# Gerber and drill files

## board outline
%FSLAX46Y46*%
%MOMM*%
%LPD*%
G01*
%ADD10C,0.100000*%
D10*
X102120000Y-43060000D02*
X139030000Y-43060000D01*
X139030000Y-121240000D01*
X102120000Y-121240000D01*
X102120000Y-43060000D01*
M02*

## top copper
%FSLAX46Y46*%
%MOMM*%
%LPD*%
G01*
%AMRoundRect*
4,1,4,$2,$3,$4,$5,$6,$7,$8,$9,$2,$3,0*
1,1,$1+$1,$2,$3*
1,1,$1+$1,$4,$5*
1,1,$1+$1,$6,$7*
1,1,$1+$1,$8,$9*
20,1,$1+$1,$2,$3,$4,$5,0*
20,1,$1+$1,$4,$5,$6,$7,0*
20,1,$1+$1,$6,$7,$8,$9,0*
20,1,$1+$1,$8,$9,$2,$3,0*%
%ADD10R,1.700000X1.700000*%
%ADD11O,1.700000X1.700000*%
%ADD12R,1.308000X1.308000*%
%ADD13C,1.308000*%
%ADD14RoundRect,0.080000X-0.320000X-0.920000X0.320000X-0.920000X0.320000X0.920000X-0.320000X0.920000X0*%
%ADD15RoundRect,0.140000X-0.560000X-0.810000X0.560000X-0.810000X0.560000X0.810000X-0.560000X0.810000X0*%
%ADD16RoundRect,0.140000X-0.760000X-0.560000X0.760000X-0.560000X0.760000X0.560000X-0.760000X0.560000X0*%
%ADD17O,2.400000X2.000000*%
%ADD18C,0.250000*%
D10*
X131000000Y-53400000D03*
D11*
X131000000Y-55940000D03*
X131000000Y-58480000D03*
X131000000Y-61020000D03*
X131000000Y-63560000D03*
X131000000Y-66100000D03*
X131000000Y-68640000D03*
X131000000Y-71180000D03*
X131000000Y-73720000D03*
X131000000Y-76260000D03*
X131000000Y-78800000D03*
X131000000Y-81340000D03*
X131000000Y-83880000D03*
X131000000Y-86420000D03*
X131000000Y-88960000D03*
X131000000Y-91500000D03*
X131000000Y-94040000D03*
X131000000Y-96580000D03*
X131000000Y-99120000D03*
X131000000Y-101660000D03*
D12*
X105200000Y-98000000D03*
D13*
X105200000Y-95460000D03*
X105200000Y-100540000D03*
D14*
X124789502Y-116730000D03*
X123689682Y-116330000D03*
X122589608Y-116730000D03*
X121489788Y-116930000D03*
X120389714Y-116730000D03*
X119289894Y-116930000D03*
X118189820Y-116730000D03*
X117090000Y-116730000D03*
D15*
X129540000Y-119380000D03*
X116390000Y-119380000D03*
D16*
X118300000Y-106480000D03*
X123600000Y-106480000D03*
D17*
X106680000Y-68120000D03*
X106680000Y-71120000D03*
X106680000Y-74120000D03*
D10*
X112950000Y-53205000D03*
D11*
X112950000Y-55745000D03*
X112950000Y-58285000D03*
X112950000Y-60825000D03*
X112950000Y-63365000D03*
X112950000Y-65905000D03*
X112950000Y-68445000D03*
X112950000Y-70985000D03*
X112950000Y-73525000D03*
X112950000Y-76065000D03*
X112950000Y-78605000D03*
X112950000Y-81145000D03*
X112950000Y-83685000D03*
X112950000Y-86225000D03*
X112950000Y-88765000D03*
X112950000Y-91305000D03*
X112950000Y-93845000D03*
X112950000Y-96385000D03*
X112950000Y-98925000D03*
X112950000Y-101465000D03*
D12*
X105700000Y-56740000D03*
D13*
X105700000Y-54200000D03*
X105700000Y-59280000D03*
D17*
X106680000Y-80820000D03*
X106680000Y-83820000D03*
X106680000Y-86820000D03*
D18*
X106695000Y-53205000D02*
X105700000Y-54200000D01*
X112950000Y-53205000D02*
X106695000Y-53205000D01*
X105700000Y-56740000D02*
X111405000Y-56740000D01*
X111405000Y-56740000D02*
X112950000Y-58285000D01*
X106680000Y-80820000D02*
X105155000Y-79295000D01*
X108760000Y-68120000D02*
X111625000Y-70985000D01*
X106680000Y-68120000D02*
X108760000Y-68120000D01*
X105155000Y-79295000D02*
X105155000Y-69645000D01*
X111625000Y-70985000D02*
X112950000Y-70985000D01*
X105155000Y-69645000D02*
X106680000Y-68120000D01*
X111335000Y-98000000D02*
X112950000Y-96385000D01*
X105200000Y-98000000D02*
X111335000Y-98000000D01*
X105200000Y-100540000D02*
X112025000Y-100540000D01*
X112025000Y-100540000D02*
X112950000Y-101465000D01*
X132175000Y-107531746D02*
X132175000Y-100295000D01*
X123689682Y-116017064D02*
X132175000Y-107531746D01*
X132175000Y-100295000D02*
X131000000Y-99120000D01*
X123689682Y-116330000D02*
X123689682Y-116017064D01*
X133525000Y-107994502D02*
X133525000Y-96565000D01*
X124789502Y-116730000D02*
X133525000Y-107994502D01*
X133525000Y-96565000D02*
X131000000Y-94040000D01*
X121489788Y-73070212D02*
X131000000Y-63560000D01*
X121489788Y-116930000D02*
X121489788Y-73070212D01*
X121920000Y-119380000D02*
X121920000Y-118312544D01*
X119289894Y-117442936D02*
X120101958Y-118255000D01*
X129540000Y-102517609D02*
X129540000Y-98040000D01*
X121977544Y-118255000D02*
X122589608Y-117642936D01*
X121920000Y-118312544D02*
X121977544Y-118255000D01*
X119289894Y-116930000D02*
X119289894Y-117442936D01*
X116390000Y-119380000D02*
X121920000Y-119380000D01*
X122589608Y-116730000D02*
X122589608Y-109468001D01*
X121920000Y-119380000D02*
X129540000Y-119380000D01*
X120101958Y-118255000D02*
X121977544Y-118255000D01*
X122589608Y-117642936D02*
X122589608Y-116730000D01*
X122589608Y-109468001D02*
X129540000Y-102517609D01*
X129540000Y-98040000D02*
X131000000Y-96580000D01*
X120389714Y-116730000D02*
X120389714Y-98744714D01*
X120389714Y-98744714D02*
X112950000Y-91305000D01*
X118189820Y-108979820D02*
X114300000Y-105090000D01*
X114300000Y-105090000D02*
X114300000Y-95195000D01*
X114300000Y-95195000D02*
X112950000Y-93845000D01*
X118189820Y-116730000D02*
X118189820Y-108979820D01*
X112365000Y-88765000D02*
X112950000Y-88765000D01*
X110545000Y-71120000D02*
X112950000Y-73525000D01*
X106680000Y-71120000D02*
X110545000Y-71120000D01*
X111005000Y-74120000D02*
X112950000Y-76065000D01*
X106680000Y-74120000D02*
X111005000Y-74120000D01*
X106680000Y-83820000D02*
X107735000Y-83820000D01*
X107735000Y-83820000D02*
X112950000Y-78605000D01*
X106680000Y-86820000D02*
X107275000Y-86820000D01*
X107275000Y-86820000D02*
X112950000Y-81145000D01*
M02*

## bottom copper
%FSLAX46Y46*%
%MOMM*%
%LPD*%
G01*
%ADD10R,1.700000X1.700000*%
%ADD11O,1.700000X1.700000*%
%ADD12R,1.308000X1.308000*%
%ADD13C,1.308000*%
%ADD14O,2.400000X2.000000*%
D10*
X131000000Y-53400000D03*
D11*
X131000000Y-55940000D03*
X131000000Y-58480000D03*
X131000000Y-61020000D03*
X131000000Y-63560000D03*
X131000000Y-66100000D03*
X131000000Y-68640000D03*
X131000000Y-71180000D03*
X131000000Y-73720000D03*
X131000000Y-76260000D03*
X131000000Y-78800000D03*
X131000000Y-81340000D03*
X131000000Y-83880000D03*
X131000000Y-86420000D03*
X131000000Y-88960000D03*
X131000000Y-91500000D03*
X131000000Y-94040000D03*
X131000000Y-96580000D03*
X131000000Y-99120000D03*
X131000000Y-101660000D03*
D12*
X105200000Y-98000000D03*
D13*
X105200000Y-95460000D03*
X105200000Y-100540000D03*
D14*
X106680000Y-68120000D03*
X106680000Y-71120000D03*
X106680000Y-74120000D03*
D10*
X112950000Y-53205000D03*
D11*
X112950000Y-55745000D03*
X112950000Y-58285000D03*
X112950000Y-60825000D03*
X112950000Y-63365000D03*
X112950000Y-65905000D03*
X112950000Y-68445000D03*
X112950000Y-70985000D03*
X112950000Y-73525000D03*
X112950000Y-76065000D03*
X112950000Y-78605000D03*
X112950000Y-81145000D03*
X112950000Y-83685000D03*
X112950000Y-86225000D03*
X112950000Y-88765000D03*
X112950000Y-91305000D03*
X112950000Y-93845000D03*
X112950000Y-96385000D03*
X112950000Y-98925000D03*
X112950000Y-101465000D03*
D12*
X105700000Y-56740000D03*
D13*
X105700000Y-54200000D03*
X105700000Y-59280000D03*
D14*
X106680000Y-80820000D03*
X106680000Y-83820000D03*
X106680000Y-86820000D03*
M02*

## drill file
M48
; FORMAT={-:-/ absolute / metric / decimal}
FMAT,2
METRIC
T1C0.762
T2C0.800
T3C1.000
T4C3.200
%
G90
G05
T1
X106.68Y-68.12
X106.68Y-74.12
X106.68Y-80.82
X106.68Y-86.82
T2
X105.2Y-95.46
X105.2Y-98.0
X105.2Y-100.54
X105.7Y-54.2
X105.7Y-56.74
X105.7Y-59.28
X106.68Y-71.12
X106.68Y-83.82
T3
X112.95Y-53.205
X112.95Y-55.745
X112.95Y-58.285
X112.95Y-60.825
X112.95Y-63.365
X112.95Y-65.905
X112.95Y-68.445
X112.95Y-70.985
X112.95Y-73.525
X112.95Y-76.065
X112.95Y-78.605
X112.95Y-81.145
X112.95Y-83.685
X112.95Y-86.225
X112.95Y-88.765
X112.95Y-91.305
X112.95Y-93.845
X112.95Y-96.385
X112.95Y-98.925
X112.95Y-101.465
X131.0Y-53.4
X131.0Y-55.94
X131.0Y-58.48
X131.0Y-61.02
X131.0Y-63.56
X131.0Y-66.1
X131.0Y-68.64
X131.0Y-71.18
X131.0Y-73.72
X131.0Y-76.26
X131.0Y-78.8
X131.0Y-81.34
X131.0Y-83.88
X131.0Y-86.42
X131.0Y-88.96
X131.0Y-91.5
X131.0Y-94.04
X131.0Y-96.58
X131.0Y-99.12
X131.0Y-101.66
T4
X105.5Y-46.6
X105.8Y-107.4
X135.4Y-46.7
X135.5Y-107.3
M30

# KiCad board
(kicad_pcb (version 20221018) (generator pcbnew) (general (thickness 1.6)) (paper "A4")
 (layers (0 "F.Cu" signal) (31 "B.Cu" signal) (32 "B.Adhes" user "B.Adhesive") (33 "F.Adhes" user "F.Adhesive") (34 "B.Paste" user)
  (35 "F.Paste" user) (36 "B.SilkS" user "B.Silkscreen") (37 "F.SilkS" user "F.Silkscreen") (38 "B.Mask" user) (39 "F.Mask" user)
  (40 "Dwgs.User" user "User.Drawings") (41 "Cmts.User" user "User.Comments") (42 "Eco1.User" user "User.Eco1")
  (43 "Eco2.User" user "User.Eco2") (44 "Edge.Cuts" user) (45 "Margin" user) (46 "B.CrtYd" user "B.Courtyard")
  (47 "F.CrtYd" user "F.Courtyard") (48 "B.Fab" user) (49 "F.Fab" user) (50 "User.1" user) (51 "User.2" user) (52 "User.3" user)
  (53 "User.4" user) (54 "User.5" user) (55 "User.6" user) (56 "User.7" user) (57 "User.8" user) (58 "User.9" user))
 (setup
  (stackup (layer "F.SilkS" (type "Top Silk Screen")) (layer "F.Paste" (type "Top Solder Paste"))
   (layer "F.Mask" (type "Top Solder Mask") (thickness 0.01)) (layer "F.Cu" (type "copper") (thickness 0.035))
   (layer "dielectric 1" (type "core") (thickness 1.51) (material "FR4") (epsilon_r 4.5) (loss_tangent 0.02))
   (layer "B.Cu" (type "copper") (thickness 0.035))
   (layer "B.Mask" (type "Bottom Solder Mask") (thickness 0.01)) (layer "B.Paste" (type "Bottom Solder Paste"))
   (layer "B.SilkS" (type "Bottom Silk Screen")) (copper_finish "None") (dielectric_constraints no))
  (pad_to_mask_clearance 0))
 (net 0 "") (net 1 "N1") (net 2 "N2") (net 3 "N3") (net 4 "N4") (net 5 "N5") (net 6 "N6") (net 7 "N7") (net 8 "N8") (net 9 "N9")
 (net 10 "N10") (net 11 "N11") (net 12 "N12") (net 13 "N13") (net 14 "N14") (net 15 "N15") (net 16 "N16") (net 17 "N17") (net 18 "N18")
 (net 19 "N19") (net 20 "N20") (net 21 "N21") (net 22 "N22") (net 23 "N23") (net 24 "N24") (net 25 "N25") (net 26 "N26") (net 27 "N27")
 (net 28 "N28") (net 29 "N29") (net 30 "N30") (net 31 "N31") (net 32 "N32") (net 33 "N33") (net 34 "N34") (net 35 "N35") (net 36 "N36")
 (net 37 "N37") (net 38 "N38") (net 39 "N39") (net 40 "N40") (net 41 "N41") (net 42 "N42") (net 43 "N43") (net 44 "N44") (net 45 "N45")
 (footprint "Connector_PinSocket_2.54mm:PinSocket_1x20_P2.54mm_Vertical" (layer "F.Cu") (at 131 53.4)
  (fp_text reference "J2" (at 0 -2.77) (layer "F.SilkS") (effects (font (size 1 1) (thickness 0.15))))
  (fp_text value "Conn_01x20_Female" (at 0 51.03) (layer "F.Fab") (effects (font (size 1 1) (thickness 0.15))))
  (pad "1" thru_hole rect (at 0 0) (size 1.7 1.7) (drill 1) (layers "*.Cu" "*.Mask") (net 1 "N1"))
  (pad "2" thru_hole oval (at 0 2.54) (size 1.7 1.7) (drill 1) (layers "*.Cu" "*.Mask") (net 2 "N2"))
  (pad "3" thru_hole oval (at 0 5.08) (size 1.7 1.7) (drill 1) (layers "*.Cu" "*.Mask") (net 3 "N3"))
  (pad "4" thru_hole oval (at 0 7.62) (size 1.7 1.7) (drill 1) (layers "*.Cu" "*.Mask") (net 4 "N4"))
  (pad "5" thru_hole oval (at 0 10.16) (size 1.7 1.7) (drill 1) (layers "*.Cu" "*.Mask") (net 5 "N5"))
  (pad "6" thru_hole oval (at 0 12.7) (size 1.7 1.7) (drill 1) (layers "*.Cu" "*.Mask") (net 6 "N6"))
  (pad "7" thru_hole oval (at 0 15.24) (size 1.7 1.7) (drill 1) (layers "*.Cu" "*.Mask") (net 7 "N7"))
  (pad "8" thru_hole oval (at 0 17.78) (size 1.7 1.7) (drill 1) (layers "*.Cu" "*.Mask") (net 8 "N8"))
  (pad "9" thru_hole oval (at 0 20.32) (size 1.7 1.7) (drill 1) (layers "*.Cu" "*.Mask") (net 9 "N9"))
  (pad "10" thru_hole oval (at 0 22.86) (size 1.7 1.7) (drill 1) (layers "*.Cu" "*.Mask") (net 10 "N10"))
  (pad "11" thru_hole oval (at 0 25.4) (size 1.7 1.7) (drill 1) (layers "*.Cu" "*.Mask") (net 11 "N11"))
  (pad "12" thru_hole oval (at 0 27.94) (size 1.7 1.7) (drill 1) (layers "*.Cu" "*.Mask") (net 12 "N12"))
  (pad "13" thru_hole oval (at 0 30.48) (size 1.7 1.7) (drill 1) (layers "*.Cu" "*.Mask") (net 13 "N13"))
  (pad "14" thru_hole oval (at 0 33.02) (size 1.7 1.7) (drill 1) (layers "*.Cu" "*.Mask") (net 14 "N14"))
  (pad "15" thru_hole oval (at 0 35.56) (size 1.7 1.7) (drill 1) (layers "*.Cu" "*.Mask") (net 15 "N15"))
  (pad "16" thru_hole oval (at 0 38.1) (size 1.7 1.7) (drill 1) (layers "*.Cu" "*.Mask") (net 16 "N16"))
  (pad "17" thru_hole oval (at 0 40.64) (size 1.7 1.7) (drill 1) (layers "*.Cu" "*.Mask") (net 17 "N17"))
  (pad "18" thru_hole oval (at 0 43.18) (size 1.7 1.7) (drill 1) (layers "*.Cu" "*.Mask") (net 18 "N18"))
  (pad "19" thru_hole oval (at 0 45.72) (size 1.7 1.7) (drill 1) (layers "*.Cu" "*.Mask") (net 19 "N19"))
  (pad "20" thru_hole oval (at 0 48.26) (size 1.7 1.7) (drill 1) (layers "*.Cu" "*.Mask") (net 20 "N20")))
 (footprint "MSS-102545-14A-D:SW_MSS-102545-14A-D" (layer "F.Cu") (at 105.2 98 -90)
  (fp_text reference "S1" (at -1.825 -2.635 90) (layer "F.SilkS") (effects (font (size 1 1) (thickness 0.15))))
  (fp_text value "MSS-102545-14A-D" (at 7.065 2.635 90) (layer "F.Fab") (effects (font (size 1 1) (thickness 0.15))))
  (pad "1" thru_hole rect (at 0 0 270) (size 1.308 1.308) (drill 0.8) (layers "*.Cu" "*.Mask") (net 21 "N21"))
  (pad "2" thru_hole circle (at -2.54 0 270) (size 1.308 1.308) (drill 0.8) (layers "*.Cu" "*.Mask") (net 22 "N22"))
  (pad "3" thru_hole circle (at 2.54 0 270) (size 1.308 1.308) (drill 0.8) (layers "*.Cu" "*.Mask") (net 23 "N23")))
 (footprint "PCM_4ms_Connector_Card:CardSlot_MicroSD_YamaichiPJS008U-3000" (layer "F.Cu") (at 121.92 117.83008)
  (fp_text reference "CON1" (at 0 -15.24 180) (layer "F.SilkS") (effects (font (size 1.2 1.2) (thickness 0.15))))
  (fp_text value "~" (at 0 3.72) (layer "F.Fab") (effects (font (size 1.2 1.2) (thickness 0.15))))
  (pad "1" smd roundrect (at 2.869502 -1.10008) (size 0.8 2) (layers "F.Cu" "F.Paste" "F.Mask") (roundrect_rratio 0.1) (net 17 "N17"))
  (pad "2" smd roundrect (at 1.769682 -1.50008) (size 0.8 2) (layers "F.Cu" "F.Paste" "F.Mask") (roundrect_rratio 0.1) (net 19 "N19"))
  (pad "3" smd roundrect (at 0.669608 -1.10008) (size 0.8 2) (layers "F.Cu" "F.Paste" "F.Mask") (roundrect_rratio 0.1) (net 18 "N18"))
  (pad "4" smd roundrect (at -0.430212 -0.90008) (size 0.8 2) (layers "F.Cu" "F.Paste" "F.Mask") (roundrect_rratio 0.1) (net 5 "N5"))
  (pad "5" smd roundrect (at -1.530286 -1.10008) (size 0.8 2) (layers "F.Cu" "F.Paste" "F.Mask") (roundrect_rratio 0.1) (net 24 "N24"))
  (pad "6" smd roundrect (at -2.630106 -0.90008) (size 0.8 2) (layers "F.Cu" "F.Paste" "F.Mask") (roundrect_rratio 0.1) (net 18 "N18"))
  (pad "7" smd roundrect (at -3.73018 -1.10008) (size 0.8 2) (layers "F.Cu" "F.Paste" "F.Mask") (roundrect_rratio 0.1) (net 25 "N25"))
  (pad "8" smd roundrect (at -4.83 -1.10008) (size 0.8 2) (layers "F.Cu" "F.Paste" "F.Mask") (roundrect_rratio 0.1) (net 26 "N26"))
  (pad "9" smd roundrect (at 7.62 1.54992) (size 1.4 1.9) (layers "F.Cu" "F.Paste" "F.Mask") (roundrect_rratio 0.1) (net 18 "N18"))
  (pad "10" smd roundrect (at -5.53 1.54992) (size 1.4 1.9) (layers "F.Cu" "F.Paste" "F.Mask") (roundrect_rratio 0.1) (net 18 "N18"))
  (pad "11" smd roundrect (at -3.62 -11.35008) (size 1.8 1.4) (layers "F.Cu" "F.Paste" "F.Mask") (roundrect_rratio 0.1))
  (pad "12" smd roundrect (at 1.68 -11.35008) (size 1.8 1.4) (layers "F.Cu" "F.Paste" "F.Mask") (roundrect_rratio 0.1)))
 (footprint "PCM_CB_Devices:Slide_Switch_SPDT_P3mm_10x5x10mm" (layer "F.Cu") (at 106.68 68.12 -90)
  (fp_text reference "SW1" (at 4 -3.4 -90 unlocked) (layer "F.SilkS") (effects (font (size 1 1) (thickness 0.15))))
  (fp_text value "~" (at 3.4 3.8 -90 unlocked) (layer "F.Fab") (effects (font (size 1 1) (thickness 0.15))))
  (pad "1" thru_hole oval (at 0 0 270) (size 2 2.4) (drill 0.762) (layers "*.Cu" "*.Mask") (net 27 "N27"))
  (pad "2" thru_hole oval (at 3 0 270) (size 2 2.4) (drill 0.8) (layers "*.Cu" "*.Mask") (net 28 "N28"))
  (pad "3" thru_hole oval (at 6 0 270) (size 2 2.4) (drill 0.762) (layers "*.Cu" "*.Mask") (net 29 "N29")))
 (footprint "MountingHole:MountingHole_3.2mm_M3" (layer "F.Cu") (at 105.5 46.6)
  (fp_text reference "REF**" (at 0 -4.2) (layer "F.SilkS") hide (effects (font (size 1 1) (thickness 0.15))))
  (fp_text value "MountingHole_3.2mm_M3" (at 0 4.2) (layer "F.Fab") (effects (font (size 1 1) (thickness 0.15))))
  (pad "" np_thru_hole circle (at 0 0) (size 3.2 3.2) (drill 3.2) (layers "*.Cu" "*.Mask")))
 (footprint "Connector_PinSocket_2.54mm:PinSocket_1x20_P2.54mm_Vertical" (layer "F.Cu") (at 112.95 53.205)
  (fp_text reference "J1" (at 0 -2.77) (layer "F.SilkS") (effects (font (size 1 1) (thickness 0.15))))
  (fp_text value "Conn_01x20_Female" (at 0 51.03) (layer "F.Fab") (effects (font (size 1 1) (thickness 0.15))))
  (pad "1" thru_hole rect (at 0 0) (size 1.7 1.7) (drill 1) (layers "*.Cu" "*.Mask") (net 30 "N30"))
  (pad "2" thru_hole oval (at 0 2.54) (size 1.7 1.7) (drill 1) (layers "*.Cu" "*.Mask") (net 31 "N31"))
  (pad "3" thru_hole oval (at 0 5.08) (size 1.7 1.7) (drill 1) (layers "*.Cu" "*.Mask") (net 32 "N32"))
  (pad "4" thru_hole oval (at 0 7.62) (size 1.7 1.7) (drill 1) (layers "*.Cu" "*.Mask") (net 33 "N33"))
  (pad "5" thru_hole oval (at 0 10.16) (size 1.7 1.7) (drill 1) (layers "*.Cu" "*.Mask") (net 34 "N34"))
  (pad "6" thru_hole oval (at 0 12.7) (size 1.7 1.7) (drill 1) (layers "*.Cu" "*.Mask") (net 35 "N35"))
  (pad "7" thru_hole oval (at 0 15.24) (size 1.7 1.7) (drill 1) (layers "*.Cu" "*.Mask") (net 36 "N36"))
  (pad "8" thru_hole oval (at 0 17.78) (size 1.7 1.7) (drill 1) (layers "*.Cu" "*.Mask") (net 27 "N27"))
  (pad "9" thru_hole oval (at 0 20.32) (size 1.7 1.7) (drill 1) (layers "*.Cu" "*.Mask") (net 28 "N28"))
  (pad "10" thru_hole oval (at 0 22.86) (size 1.7 1.7) (drill 1) (layers "*.Cu" "*.Mask") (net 29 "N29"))
  (pad "11" thru_hole oval (at 0 25.4) (size 1.7 1.7) (drill 1) (layers "*.Cu" "*.Mask") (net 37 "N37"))
  (pad "12" thru_hole oval (at 0 27.94) (size 1.7 1.7) (drill 1) (layers "*.Cu" "*.Mask") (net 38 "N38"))
  (pad "13" thru_hole oval (at 0 30.48) (size 1.7 1.7) (drill 1) (layers "*.Cu" "*.Mask") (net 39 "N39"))
  (pad "14" thru_hole oval (at 0 33.02) (size 1.7 1.7) (drill 1) (layers "*.Cu" "*.Mask") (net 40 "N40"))
  (pad "15" thru_hole oval (at 0 35.56) (size 1.7 1.7) (drill 1) (layers "*.Cu" "*.Mask") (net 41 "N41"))
  (pad "16" thru_hole oval (at 0 38.1) (size 1.7 1.7) (drill 1) (layers "*.Cu" "*.Mask") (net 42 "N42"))
  (pad "17" thru_hole oval (at 0 40.64) (size 1.7 1.7) (drill 1) (layers "*.Cu" "*.Mask") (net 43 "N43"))
  (pad "18" thru_hole oval (at 0 43.18) (size 1.7 1.7) (drill 1) (layers "*.Cu" "*.Mask") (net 21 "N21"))
  (pad "19" thru_hole oval (at 0 45.72) (size 1.7 1.7) (drill 1) (layers "*.Cu" "*.Mask") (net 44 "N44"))
  (pad "20" thru_hole oval (at 0 48.26) (size 1.7 1.7) (drill 1) (layers "*.Cu" "*.Mask") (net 23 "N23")))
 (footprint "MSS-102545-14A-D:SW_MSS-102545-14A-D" (layer "F.Cu") (at 105.7 56.74 -90)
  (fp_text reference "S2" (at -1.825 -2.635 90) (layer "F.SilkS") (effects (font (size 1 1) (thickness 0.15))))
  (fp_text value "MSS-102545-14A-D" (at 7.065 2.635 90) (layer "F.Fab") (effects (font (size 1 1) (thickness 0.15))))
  (pad "1" thru_hole rect (at 0 0 270) (size 1.308 1.308) (drill 0.8) (layers "*.Cu" "*.Mask") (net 32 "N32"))
  (pad "2" thru_hole circle (at -2.54 0 270) (size 1.308 1.308) (drill 0.8) (layers "*.Cu" "*.Mask") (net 30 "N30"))
  (pad "3" thru_hole circle (at 2.54 0 270) (size 1.308 1.308) (drill 0.8) (layers "*.Cu" "*.Mask") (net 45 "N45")))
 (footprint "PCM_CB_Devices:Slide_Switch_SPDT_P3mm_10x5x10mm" (layer "F.Cu") (at 106.68 80.82 -90)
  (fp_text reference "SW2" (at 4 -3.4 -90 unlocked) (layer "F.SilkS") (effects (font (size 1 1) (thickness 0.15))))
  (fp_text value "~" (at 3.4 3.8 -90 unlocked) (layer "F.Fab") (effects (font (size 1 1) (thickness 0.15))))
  (pad "1" thru_hole oval (at 0 0 270) (size 2 2.4) (drill 0.762) (layers "*.Cu" "*.Mask") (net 27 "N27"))
  (pad "2" thru_hole oval (at 3 0 270) (size 2 2.4) (drill 0.8) (layers "*.Cu" "*.Mask") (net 37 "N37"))
  (pad "3" thru_hole oval (at 6 0 270) (size 2 2.4) (drill 0.762) (layers "*.Cu" "*.Mask") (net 38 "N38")))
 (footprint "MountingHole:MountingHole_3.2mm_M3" (layer "F.Cu") (at 135.4 46.7)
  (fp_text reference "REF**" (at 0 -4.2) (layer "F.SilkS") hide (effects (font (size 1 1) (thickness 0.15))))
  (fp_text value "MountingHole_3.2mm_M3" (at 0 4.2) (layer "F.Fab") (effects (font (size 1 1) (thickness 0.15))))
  (pad "" np_thru_hole circle (at 0 0) (size 3.2 3.2) (drill 3.2) (layers "*.Cu" "*.Mask")))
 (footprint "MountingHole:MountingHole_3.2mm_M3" (layer "F.Cu") (at 135.5 107.3)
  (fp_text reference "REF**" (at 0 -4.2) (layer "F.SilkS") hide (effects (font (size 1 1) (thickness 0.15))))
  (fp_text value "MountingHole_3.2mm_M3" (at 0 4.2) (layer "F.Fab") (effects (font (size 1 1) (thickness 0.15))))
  (pad "" np_thru_hole circle (at 0 0) (size 3.2 3.2) (drill 3.2) (layers "*.Cu" "*.Mask")))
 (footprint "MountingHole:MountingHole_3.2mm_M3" (layer "F.Cu") (at 105.8 107.4)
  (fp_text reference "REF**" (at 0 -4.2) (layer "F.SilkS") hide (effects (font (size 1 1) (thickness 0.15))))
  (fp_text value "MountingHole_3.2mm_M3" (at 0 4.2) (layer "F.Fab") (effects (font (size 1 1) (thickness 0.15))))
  (pad "" np_thru_hole circle (at 0 0) (size 3.2 3.2) (drill 3.2) (layers "*.Cu" "*.Mask")))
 (gr_rect (start 102.12 43.06) (end 139.03 121.24) (stroke (width 0.1) (type solid)) (fill none) (layer "Edge.Cuts"))
 (segment (start 106.695 53.205) (end 105.7 54.2) (width 0.25) (layer "F.Cu") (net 30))
 (segment (start 112.95 53.205) (end 106.695 53.205) (width 0.25) (layer "F.Cu") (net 30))
 (segment (start 105.7 56.74) (end 111.405 56.74) (width 0.25) (layer "F.Cu") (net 32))
 (segment (start 111.405 56.74) (end 112.95 58.285) (width 0.25) (layer "F.Cu") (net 32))
 (segment (start 106.68 80.82) (end 105.155 79.295) (width 0.25) (layer "F.Cu") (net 27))
 (segment (start 108.76 68.12) (end 111.625 70.985) (width 0.25) (layer "F.Cu") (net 27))
 (segment (start 106.68 68.12) (end 108.76 68.12) (width 0.25) (layer "F.Cu") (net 27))
 (segment (start 105.155 79.295) (end 105.155 69.645) (width 0.25) (layer "F.Cu") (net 27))
 (segment (start 111.625 70.985) (end 112.95 70.985) (width 0.25) (layer "F.Cu") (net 27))
 (segment (start 105.155 69.645) (end 106.68 68.12) (width 0.25) (layer "F.Cu") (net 27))
 (segment (start 111.335 98) (end 112.95 96.385) (width 0.25) (layer "F.Cu") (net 21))
 (segment (start 105.2 98) (end 111.335 98) (width 0.25) (layer "F.Cu") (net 21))
 (segment (start 105.2 100.54) (end 112.025 100.54) (width 0.25) (layer "F.Cu") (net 23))
 (segment (start 112.025 100.54) (end 112.95 101.465) (width 0.25) (layer "F.Cu") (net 23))
 (segment (start 132.175 107.531746) (end 132.175 100.295) (width 0.25) (layer "F.Cu") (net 19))
 (segment (start 123.689682 116.017064) (end 132.175 107.531746) (width 0.25) (layer "F.Cu") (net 19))
 (segment (start 132.175 100.295) (end 131 99.12) (width 0.25) (layer "F.Cu") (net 19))
 (segment (start 123.689682 116.33) (end 123.689682 116.017064) (width 0.25) (layer "F.Cu") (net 19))
 (segment (start 133.525 107.994502) (end 133.525 96.565) (width 0.25) (layer "F.Cu") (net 17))
 (segment (start 124.789502 116.73) (end 133.525 107.994502) (width 0.25) (layer "F.Cu") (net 17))
 (segment (start 133.525 96.565) (end 131 94.04) (width 0.25) (layer "F.Cu") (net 17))
 (segment (start 121.489788 73.070212) (end 131 63.56) (width 0.25) (layer "F.Cu") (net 5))
 (segment (start 121.489788 116.93) (end 121.489788 73.070212) (width 0.25) (layer "F.Cu") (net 5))
 (segment (start 121.92 119.38) (end 121.92 118.312544) (width 0.25) (layer "F.Cu") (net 18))
 (segment (start 119.289894 117.442936) (end 120.101958 118.255) (width 0.25) (layer "F.Cu") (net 18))
 (segment (start 129.54 102.517609) (end 129.54 98.04) (width 0.25) (layer "F.Cu") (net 18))
 (segment (start 121.977544 118.255) (end 122.589608 117.642936) (width 0.25) (layer "F.Cu") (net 18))
 (segment (start 121.92 118.312544) (end 121.977544 118.255) (width 0.25) (layer "F.Cu") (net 18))
 (segment (start 119.289894 116.93) (end 119.289894 117.442936) (width 0.25) (layer "F.Cu") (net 18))
 (segment (start 116.39 119.38) (end 121.92 119.38) (width 0.25) (layer "F.Cu") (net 18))
 (segment (start 122.589608 116.73) (end 122.589608 109.468001) (width 0.25) (layer "F.Cu") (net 18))
 (segment (start 121.92 119.38) (end 129.54 119.38) (width 0.25) (layer "F.Cu") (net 18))
 (segment (start 120.101958 118.255) (end 121.977544 118.255) (width 0.25) (layer "F.Cu") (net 18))
 (segment (start 122.589608 117.642936) (end 122.589608 116.73) (width 0.25) (layer "F.Cu") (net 18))
 (segment (start 122.589608 109.468001) (end 129.54 102.517609) (width 0.25) (layer "F.Cu") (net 18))
 (segment (start 129.54 98.04) (end 131 96.58) (width 0.25) (layer "F.Cu") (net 18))
 (segment (start 120.389714 116.73) (end 120.389714 98.744714) (width 0.25) (layer "F.Cu") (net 24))
 (segment (start 120.389714 98.744714) (end 112.95 91.305) (width 0.25) (layer "F.Cu") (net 24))
 (segment (start 118.18982 108.97982) (end 114.3 105.09) (width 0.25) (layer "F.Cu") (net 25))
 (segment (start 114.3 105.09) (end 114.3 95.195) (width 0.25) (layer "F.Cu") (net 25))
 (segment (start 114.3 95.195) (end 112.95 93.845) (width 0.25) (layer "F.Cu") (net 25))
 (segment (start 118.18982 116.73) (end 118.18982 108.97982) (width 0.25) (layer "F.Cu") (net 25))
 (segment (start 112.365 88.765) (end 112.95 88.765) (width 0.25) (layer "F.Cu") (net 41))
 (segment (start 110.545 71.12) (end 112.95 73.525) (width 0.25) (layer "F.Cu") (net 28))
 (segment (start 106.68 71.12) (end 110.545 71.12) (width 0.25) (layer "F.Cu") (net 28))
 (segment (start 111.005 74.12) (end 112.95 76.065) (width 0.25) (layer "F.Cu") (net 29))
 (segment (start 106.68 74.12) (end 111.005 74.12) (width 0.25) (layer "F.Cu") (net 29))
 (segment (start 106.68 83.82) (end 107.735 83.82) (width 0.25) (layer "F.Cu") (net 37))
 (segment (start 107.735 83.82) (end 112.95 78.605) (width 0.25) (layer "F.Cu") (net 37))
 (segment (start 106.68 86.82) (end 107.275 86.82) (width 0.25) (layer "F.Cu") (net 38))
 (segment (start 107.275 86.82) (end 112.95 81.145) (width 0.25) (layer "F.Cu") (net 38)))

